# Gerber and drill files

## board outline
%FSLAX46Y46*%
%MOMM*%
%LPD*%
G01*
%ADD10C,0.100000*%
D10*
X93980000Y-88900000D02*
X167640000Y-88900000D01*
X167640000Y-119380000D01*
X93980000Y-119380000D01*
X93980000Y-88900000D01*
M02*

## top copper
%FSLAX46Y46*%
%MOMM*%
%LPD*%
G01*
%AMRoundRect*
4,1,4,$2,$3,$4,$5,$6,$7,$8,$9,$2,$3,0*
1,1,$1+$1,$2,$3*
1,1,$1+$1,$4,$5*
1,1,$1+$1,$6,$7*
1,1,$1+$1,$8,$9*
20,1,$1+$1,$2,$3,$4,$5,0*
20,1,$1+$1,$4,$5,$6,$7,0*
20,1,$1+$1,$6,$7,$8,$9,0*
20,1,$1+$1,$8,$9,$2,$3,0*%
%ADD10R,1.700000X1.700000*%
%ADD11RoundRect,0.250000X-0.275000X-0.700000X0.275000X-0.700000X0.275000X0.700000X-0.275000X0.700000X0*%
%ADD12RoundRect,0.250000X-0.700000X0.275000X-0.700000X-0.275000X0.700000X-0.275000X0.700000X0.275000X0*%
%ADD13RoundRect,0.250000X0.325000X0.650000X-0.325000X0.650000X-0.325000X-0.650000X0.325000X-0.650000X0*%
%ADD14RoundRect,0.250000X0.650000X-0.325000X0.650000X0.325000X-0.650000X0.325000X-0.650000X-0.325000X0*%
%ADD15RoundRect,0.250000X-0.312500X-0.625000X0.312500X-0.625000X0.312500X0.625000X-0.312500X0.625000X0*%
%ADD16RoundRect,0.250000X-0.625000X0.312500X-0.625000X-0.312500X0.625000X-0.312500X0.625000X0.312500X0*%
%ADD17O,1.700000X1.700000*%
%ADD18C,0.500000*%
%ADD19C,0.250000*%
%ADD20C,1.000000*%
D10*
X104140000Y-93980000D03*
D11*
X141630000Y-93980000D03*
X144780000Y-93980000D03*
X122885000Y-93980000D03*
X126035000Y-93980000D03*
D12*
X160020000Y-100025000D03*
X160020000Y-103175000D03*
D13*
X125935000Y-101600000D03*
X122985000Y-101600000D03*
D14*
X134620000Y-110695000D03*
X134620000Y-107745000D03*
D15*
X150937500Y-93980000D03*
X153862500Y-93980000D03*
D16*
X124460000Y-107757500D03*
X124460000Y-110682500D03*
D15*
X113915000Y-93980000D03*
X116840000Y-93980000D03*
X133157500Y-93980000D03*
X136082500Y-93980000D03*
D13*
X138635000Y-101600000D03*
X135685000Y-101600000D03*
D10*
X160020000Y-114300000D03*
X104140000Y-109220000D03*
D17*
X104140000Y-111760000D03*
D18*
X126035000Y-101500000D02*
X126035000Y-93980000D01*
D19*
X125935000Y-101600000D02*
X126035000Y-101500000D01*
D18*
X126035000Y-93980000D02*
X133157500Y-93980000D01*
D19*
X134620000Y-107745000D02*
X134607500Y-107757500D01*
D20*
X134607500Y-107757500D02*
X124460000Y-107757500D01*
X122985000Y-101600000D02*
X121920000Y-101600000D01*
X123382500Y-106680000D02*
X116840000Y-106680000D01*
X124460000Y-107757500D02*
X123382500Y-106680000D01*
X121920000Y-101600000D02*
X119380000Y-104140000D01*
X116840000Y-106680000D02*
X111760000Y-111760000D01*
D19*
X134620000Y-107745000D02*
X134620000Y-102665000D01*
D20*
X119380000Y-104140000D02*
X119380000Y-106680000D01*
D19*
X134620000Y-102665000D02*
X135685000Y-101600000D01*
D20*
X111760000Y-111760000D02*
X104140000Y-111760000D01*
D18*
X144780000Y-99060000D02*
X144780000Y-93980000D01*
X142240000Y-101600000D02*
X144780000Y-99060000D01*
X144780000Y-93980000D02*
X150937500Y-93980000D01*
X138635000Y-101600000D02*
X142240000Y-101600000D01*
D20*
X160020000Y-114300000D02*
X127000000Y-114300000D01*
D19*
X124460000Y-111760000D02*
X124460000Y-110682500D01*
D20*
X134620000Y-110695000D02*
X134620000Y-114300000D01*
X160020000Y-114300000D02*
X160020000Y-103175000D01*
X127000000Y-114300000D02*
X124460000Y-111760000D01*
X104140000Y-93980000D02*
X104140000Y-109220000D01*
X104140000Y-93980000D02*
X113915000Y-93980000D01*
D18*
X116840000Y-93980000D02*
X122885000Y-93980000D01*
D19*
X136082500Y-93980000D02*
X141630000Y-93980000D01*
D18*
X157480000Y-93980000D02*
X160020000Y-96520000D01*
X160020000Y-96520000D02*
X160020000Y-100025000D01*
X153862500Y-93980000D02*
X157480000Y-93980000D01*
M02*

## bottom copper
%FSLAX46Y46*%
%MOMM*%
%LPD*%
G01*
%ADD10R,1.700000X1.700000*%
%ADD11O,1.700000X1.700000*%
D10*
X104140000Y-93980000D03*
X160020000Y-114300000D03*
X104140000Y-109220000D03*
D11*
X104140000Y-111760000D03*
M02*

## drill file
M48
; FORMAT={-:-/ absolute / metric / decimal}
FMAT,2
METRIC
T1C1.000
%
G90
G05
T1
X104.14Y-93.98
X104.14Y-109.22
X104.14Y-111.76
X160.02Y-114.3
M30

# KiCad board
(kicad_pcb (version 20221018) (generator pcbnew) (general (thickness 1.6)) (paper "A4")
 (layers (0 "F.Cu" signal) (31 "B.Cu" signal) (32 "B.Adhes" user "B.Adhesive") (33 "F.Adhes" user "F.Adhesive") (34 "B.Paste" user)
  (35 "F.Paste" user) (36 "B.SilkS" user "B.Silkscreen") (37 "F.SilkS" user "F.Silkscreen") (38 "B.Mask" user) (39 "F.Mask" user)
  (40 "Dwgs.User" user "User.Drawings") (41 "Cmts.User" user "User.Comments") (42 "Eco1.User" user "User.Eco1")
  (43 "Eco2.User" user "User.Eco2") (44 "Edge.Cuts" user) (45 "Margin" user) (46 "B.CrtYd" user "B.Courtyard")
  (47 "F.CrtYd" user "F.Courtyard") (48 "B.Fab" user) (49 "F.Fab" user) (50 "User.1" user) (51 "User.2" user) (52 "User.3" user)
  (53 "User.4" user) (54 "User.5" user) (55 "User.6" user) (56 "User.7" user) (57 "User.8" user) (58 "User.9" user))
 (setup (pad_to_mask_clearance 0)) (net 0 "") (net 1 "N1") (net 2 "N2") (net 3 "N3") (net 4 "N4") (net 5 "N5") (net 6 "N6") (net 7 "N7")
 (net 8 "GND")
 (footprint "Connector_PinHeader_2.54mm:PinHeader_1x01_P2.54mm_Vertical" (layer "F.Cu") (at 104.14 93.98)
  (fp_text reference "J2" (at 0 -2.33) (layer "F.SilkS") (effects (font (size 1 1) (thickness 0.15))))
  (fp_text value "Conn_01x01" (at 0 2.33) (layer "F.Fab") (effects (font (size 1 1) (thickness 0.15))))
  (pad "1" thru_hole rect (at 0 0) (size 1.7 1.7) (drill 1) (layers "*.Cu" "*.Mask") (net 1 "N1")))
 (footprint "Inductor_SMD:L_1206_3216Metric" (layer "F.Cu") (at 143.205 93.98)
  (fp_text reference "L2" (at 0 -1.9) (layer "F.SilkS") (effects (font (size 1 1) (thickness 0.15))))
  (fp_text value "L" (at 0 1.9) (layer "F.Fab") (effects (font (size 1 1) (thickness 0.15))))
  (pad "1" smd roundrect (at -1.575 0) (size 1.05 1.9) (layers "F.Cu" "F.Paste" "F.Mask") (roundrect_rratio 0.238095) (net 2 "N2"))
  (pad "2" smd roundrect (at 1.575 0) (size 1.05 1.9) (layers "F.Cu" "F.Paste" "F.Mask") (roundrect_rratio 0.238095) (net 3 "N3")))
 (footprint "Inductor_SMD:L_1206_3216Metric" (layer "F.Cu") (at 124.46 93.98)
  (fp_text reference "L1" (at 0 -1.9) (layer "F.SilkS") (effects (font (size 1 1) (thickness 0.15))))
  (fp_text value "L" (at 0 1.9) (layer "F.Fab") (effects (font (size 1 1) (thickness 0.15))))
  (pad "1" smd roundrect (at -1.575 0) (size 1.05 1.9) (layers "F.Cu" "F.Paste" "F.Mask") (roundrect_rratio 0.238095) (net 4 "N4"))
  (pad "2" smd roundrect (at 1.575 0) (size 1.05 1.9) (layers "F.Cu" "F.Paste" "F.Mask") (roundrect_rratio 0.238095) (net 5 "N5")))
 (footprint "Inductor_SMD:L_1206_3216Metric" (layer "F.Cu") (at 160.02 101.6 -90)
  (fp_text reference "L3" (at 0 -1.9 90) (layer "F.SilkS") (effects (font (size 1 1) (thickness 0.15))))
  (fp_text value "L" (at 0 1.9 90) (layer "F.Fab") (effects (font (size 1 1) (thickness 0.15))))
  (pad "1" smd roundrect (at -1.575 0 270) (size 1.05 1.9) (layers "F.Cu" "F.Paste" "F.Mask") (roundrect_rratio 0.238095) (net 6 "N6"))
  (pad "2" smd roundrect (at 1.575 0 270) (size 1.05 1.9) (layers "F.Cu" "F.Paste" "F.Mask") (roundrect_rratio 0.238095) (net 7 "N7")))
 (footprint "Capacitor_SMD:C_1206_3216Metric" (layer "F.Cu") (at 124.46 101.6 180)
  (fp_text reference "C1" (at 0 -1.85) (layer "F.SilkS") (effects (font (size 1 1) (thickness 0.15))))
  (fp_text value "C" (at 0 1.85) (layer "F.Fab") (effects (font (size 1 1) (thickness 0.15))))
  (pad "1" smd roundrect (at -1.475 0 180) (size 1.15 1.8) (layers "F.Cu" "F.Paste" "F.Mask") (roundrect_rratio 0.217391) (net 5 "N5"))
  (pad "2" smd roundrect (at 1.475 0 180) (size 1.15 1.8) (layers "F.Cu" "F.Paste" "F.Mask") (roundrect_rratio 0.217391) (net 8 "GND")))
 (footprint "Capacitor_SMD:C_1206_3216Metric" (layer "F.Cu") (at 134.62 109.22 90)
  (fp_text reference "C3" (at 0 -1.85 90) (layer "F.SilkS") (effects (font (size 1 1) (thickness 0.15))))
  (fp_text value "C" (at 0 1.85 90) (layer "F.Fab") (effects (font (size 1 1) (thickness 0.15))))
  (pad "1" smd roundrect (at -1.475 0 90) (size 1.15 1.8) (layers "F.Cu" "F.Paste" "F.Mask") (roundrect_rratio 0.217391) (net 7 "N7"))
  (pad "2" smd roundrect (at 1.475 0 90) (size 1.15 1.8) (layers "F.Cu" "F.Paste" "F.Mask") (roundrect_rratio 0.217391) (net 8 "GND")))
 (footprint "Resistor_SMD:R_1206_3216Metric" (layer "F.Cu") (at 152.4 93.98)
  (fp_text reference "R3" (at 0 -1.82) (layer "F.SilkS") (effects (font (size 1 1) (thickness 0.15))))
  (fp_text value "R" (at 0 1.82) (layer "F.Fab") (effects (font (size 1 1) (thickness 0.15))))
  (pad "1" smd roundrect (at -1.4625 0) (size 1.125 1.75) (layers "F.Cu" "F.Paste" "F.Mask") (roundrect_rratio 0.222222) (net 3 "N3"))
  (pad "2" smd roundrect (at 1.4625 0) (size 1.125 1.75) (layers "F.Cu" "F.Paste" "F.Mask") (roundrect_rratio 0.222222) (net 6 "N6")))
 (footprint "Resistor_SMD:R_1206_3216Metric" (layer "F.Cu") (at 124.46 109.22 -90)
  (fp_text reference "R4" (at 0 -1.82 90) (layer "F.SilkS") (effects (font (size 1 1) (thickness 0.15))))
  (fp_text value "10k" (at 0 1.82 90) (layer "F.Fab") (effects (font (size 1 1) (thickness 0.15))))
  (pad "1" smd roundrect (at -1.4625 0 270) (size 1.125 1.75) (layers "F.Cu" "F.Paste" "F.Mask") (roundrect_rratio 0.222222) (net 8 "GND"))
  (pad "2" smd roundrect (at 1.4625 0 270) (size 1.125 1.75) (layers "F.Cu" "F.Paste" "F.Mask") (roundrect_rratio 0.222222) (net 7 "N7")))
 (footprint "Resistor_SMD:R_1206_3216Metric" (layer "F.Cu") (at 115.3775 93.98)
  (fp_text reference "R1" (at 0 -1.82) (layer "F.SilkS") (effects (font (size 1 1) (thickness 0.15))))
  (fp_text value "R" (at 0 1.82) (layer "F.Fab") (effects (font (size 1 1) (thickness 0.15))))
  (pad "1" smd roundrect (at -1.4625 0) (size 1.125 1.75) (layers "F.Cu" "F.Paste" "F.Mask") (roundrect_rratio 0.222222) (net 1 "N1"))
  (pad "2" smd roundrect (at 1.4625 0) (size 1.125 1.75) (layers "F.Cu" "F.Paste" "F.Mask") (roundrect_rratio 0.222222) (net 4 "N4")))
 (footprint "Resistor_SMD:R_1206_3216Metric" (layer "F.Cu") (at 134.62 93.98)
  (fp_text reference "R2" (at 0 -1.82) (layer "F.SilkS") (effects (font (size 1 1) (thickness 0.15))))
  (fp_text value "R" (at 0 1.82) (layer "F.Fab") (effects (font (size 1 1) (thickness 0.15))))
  (pad "1" smd roundrect (at -1.4625 0) (size 1.125 1.75) (layers "F.Cu" "F.Paste" "F.Mask") (roundrect_rratio 0.222222) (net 5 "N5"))
  (pad "2" smd roundrect (at 1.4625 0) (size 1.125 1.75) (layers "F.Cu" "F.Paste" "F.Mask") (roundrect_rratio 0.222222) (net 2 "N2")))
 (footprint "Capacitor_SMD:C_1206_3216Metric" (layer "F.Cu") (at 137.16 101.6 180)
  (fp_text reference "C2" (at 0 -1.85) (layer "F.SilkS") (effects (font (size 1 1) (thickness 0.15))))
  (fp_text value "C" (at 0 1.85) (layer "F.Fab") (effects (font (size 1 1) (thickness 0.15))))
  (pad "1" smd roundrect (at -1.475 0 180) (size 1.15 1.8) (layers "F.Cu" "F.Paste" "F.Mask") (roundrect_rratio 0.217391) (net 3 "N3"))
  (pad "2" smd roundrect (at 1.475 0 180) (size 1.15 1.8) (layers "F.Cu" "F.Paste" "F.Mask") (roundrect_rratio 0.217391) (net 8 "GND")))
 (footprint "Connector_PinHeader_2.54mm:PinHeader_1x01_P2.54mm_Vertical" (layer "F.Cu") (at 160.02 114.3)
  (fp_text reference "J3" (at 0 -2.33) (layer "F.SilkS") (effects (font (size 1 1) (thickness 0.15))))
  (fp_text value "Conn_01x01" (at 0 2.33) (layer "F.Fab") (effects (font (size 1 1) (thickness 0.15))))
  (pad "1" thru_hole rect (at 0 0) (size 1.7 1.7) (drill 1) (layers "*.Cu" "*.Mask") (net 7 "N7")))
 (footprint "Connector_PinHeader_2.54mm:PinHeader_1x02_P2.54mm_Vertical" (layer "F.Cu") (at 104.14 109.22)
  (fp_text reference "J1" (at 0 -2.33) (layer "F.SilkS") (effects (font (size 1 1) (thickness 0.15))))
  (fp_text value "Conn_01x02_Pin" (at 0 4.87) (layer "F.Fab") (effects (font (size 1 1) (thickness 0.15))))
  (pad "1" thru_hole rect (at 0 0) (size 1.7 1.7) (drill 1) (layers "*.Cu" "*.Mask") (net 1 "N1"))
  (pad "2" thru_hole oval (at 0 2.54) (size 1.7 1.7) (drill 1) (layers "*.Cu" "*.Mask") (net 8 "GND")))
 (gr_rect (start 93.98 88.9) (end 167.64 119.38) (stroke (width 0.1) (type default)) (fill none) (layer "Edge.Cuts"))
 (segment (start 126.035 101.5) (end 126.035 93.98) (width 0.5) (layer "F.Cu") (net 5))
 (segment (start 125.935 101.6) (end 126.035 101.5) (width 0.25) (layer "F.Cu") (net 5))
 (segment (start 126.035 93.98) (end 133.1575 93.98) (width 0.5) (layer "F.Cu") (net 5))
 (segment (start 134.62 107.745) (end 134.6075 107.7575) (width 0.25) (layer "F.Cu") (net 8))
 (segment (start 134.6075 107.7575) (end 124.46 107.7575) (width 1) (layer "F.Cu") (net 8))
 (segment (start 122.985 101.6) (end 121.92 101.6) (width 1) (layer "F.Cu") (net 8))
 (segment (start 123.3825 106.68) (end 116.84 106.68) (width 1) (layer "F.Cu") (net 8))
 (segment (start 124.46 107.7575) (end 123.3825 106.68) (width 1) (layer "F.Cu") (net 8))
 (segment (start 121.92 101.6) (end 119.38 104.14) (width 1) (layer "F.Cu") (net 8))
 (segment (start 116.84 106.68) (end 111.76 111.76) (width 1) (layer "F.Cu") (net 8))
 (segment (start 134.62 107.745) (end 134.62 102.665) (width 0.25) (layer "F.Cu") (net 8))
 (segment (start 119.38 104.14) (end 119.38 106.68) (width 1) (layer "F.Cu") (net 8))
 (segment (start 134.62 102.665) (end 135.685 101.6) (width 0.25) (layer "F.Cu") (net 8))
 (segment (start 111.76 111.76) (end 104.14 111.76) (width 1) (layer "F.Cu") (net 8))
 (segment (start 144.78 99.06) (end 144.78 93.98) (width 0.5) (layer "F.Cu") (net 3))
 (segment (start 142.24 101.6) (end 144.78 99.06) (width 0.5) (layer "F.Cu") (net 3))
 (segment (start 144.78 93.98) (end 150.9375 93.98) (width 0.5) (layer "F.Cu") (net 3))
 (segment (start 138.635 101.6) (end 142.24 101.6) (width 0.5) (layer "F.Cu") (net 3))
 (segment (start 160.02 114.3) (end 127 114.3) (width 1) (layer "F.Cu") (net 7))
 (segment (start 124.46 111.76) (end 124.46 110.6825) (width 0.25) (layer "F.Cu") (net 7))
 (segment (start 134.62 110.695) (end 134.62 114.3) (width 1) (layer "F.Cu") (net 7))
 (segment (start 160.02 114.3) (end 160.02 103.175) (width 1) (layer "F.Cu") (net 7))
 (segment (start 127 114.3) (end 124.46 111.76) (width 1) (layer "F.Cu") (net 7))
 (segment (start 104.14 93.98) (end 104.14 109.22) (width 1) (layer "F.Cu") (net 1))
 (segment (start 104.14 93.98) (end 113.915 93.98) (width 1) (layer "F.Cu") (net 1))
 (segment (start 116.84 93.98) (end 122.885 93.98) (width 0.5) (layer "F.Cu") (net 4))
 (segment (start 136.0825 93.98) (end 141.63 93.98) (width 0.25) (layer "F.Cu") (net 2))
 (segment (start 157.48 93.98) (end 160.02 96.52) (width 0.5) (layer "F.Cu") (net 6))
 (segment (start 160.02 96.52) (end 160.02 100.025) (width 0.5) (layer "F.Cu") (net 6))
 (segment (start 153.8625 93.98) (end 157.48 93.98) (width 0.5) (layer "F.Cu") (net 6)))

